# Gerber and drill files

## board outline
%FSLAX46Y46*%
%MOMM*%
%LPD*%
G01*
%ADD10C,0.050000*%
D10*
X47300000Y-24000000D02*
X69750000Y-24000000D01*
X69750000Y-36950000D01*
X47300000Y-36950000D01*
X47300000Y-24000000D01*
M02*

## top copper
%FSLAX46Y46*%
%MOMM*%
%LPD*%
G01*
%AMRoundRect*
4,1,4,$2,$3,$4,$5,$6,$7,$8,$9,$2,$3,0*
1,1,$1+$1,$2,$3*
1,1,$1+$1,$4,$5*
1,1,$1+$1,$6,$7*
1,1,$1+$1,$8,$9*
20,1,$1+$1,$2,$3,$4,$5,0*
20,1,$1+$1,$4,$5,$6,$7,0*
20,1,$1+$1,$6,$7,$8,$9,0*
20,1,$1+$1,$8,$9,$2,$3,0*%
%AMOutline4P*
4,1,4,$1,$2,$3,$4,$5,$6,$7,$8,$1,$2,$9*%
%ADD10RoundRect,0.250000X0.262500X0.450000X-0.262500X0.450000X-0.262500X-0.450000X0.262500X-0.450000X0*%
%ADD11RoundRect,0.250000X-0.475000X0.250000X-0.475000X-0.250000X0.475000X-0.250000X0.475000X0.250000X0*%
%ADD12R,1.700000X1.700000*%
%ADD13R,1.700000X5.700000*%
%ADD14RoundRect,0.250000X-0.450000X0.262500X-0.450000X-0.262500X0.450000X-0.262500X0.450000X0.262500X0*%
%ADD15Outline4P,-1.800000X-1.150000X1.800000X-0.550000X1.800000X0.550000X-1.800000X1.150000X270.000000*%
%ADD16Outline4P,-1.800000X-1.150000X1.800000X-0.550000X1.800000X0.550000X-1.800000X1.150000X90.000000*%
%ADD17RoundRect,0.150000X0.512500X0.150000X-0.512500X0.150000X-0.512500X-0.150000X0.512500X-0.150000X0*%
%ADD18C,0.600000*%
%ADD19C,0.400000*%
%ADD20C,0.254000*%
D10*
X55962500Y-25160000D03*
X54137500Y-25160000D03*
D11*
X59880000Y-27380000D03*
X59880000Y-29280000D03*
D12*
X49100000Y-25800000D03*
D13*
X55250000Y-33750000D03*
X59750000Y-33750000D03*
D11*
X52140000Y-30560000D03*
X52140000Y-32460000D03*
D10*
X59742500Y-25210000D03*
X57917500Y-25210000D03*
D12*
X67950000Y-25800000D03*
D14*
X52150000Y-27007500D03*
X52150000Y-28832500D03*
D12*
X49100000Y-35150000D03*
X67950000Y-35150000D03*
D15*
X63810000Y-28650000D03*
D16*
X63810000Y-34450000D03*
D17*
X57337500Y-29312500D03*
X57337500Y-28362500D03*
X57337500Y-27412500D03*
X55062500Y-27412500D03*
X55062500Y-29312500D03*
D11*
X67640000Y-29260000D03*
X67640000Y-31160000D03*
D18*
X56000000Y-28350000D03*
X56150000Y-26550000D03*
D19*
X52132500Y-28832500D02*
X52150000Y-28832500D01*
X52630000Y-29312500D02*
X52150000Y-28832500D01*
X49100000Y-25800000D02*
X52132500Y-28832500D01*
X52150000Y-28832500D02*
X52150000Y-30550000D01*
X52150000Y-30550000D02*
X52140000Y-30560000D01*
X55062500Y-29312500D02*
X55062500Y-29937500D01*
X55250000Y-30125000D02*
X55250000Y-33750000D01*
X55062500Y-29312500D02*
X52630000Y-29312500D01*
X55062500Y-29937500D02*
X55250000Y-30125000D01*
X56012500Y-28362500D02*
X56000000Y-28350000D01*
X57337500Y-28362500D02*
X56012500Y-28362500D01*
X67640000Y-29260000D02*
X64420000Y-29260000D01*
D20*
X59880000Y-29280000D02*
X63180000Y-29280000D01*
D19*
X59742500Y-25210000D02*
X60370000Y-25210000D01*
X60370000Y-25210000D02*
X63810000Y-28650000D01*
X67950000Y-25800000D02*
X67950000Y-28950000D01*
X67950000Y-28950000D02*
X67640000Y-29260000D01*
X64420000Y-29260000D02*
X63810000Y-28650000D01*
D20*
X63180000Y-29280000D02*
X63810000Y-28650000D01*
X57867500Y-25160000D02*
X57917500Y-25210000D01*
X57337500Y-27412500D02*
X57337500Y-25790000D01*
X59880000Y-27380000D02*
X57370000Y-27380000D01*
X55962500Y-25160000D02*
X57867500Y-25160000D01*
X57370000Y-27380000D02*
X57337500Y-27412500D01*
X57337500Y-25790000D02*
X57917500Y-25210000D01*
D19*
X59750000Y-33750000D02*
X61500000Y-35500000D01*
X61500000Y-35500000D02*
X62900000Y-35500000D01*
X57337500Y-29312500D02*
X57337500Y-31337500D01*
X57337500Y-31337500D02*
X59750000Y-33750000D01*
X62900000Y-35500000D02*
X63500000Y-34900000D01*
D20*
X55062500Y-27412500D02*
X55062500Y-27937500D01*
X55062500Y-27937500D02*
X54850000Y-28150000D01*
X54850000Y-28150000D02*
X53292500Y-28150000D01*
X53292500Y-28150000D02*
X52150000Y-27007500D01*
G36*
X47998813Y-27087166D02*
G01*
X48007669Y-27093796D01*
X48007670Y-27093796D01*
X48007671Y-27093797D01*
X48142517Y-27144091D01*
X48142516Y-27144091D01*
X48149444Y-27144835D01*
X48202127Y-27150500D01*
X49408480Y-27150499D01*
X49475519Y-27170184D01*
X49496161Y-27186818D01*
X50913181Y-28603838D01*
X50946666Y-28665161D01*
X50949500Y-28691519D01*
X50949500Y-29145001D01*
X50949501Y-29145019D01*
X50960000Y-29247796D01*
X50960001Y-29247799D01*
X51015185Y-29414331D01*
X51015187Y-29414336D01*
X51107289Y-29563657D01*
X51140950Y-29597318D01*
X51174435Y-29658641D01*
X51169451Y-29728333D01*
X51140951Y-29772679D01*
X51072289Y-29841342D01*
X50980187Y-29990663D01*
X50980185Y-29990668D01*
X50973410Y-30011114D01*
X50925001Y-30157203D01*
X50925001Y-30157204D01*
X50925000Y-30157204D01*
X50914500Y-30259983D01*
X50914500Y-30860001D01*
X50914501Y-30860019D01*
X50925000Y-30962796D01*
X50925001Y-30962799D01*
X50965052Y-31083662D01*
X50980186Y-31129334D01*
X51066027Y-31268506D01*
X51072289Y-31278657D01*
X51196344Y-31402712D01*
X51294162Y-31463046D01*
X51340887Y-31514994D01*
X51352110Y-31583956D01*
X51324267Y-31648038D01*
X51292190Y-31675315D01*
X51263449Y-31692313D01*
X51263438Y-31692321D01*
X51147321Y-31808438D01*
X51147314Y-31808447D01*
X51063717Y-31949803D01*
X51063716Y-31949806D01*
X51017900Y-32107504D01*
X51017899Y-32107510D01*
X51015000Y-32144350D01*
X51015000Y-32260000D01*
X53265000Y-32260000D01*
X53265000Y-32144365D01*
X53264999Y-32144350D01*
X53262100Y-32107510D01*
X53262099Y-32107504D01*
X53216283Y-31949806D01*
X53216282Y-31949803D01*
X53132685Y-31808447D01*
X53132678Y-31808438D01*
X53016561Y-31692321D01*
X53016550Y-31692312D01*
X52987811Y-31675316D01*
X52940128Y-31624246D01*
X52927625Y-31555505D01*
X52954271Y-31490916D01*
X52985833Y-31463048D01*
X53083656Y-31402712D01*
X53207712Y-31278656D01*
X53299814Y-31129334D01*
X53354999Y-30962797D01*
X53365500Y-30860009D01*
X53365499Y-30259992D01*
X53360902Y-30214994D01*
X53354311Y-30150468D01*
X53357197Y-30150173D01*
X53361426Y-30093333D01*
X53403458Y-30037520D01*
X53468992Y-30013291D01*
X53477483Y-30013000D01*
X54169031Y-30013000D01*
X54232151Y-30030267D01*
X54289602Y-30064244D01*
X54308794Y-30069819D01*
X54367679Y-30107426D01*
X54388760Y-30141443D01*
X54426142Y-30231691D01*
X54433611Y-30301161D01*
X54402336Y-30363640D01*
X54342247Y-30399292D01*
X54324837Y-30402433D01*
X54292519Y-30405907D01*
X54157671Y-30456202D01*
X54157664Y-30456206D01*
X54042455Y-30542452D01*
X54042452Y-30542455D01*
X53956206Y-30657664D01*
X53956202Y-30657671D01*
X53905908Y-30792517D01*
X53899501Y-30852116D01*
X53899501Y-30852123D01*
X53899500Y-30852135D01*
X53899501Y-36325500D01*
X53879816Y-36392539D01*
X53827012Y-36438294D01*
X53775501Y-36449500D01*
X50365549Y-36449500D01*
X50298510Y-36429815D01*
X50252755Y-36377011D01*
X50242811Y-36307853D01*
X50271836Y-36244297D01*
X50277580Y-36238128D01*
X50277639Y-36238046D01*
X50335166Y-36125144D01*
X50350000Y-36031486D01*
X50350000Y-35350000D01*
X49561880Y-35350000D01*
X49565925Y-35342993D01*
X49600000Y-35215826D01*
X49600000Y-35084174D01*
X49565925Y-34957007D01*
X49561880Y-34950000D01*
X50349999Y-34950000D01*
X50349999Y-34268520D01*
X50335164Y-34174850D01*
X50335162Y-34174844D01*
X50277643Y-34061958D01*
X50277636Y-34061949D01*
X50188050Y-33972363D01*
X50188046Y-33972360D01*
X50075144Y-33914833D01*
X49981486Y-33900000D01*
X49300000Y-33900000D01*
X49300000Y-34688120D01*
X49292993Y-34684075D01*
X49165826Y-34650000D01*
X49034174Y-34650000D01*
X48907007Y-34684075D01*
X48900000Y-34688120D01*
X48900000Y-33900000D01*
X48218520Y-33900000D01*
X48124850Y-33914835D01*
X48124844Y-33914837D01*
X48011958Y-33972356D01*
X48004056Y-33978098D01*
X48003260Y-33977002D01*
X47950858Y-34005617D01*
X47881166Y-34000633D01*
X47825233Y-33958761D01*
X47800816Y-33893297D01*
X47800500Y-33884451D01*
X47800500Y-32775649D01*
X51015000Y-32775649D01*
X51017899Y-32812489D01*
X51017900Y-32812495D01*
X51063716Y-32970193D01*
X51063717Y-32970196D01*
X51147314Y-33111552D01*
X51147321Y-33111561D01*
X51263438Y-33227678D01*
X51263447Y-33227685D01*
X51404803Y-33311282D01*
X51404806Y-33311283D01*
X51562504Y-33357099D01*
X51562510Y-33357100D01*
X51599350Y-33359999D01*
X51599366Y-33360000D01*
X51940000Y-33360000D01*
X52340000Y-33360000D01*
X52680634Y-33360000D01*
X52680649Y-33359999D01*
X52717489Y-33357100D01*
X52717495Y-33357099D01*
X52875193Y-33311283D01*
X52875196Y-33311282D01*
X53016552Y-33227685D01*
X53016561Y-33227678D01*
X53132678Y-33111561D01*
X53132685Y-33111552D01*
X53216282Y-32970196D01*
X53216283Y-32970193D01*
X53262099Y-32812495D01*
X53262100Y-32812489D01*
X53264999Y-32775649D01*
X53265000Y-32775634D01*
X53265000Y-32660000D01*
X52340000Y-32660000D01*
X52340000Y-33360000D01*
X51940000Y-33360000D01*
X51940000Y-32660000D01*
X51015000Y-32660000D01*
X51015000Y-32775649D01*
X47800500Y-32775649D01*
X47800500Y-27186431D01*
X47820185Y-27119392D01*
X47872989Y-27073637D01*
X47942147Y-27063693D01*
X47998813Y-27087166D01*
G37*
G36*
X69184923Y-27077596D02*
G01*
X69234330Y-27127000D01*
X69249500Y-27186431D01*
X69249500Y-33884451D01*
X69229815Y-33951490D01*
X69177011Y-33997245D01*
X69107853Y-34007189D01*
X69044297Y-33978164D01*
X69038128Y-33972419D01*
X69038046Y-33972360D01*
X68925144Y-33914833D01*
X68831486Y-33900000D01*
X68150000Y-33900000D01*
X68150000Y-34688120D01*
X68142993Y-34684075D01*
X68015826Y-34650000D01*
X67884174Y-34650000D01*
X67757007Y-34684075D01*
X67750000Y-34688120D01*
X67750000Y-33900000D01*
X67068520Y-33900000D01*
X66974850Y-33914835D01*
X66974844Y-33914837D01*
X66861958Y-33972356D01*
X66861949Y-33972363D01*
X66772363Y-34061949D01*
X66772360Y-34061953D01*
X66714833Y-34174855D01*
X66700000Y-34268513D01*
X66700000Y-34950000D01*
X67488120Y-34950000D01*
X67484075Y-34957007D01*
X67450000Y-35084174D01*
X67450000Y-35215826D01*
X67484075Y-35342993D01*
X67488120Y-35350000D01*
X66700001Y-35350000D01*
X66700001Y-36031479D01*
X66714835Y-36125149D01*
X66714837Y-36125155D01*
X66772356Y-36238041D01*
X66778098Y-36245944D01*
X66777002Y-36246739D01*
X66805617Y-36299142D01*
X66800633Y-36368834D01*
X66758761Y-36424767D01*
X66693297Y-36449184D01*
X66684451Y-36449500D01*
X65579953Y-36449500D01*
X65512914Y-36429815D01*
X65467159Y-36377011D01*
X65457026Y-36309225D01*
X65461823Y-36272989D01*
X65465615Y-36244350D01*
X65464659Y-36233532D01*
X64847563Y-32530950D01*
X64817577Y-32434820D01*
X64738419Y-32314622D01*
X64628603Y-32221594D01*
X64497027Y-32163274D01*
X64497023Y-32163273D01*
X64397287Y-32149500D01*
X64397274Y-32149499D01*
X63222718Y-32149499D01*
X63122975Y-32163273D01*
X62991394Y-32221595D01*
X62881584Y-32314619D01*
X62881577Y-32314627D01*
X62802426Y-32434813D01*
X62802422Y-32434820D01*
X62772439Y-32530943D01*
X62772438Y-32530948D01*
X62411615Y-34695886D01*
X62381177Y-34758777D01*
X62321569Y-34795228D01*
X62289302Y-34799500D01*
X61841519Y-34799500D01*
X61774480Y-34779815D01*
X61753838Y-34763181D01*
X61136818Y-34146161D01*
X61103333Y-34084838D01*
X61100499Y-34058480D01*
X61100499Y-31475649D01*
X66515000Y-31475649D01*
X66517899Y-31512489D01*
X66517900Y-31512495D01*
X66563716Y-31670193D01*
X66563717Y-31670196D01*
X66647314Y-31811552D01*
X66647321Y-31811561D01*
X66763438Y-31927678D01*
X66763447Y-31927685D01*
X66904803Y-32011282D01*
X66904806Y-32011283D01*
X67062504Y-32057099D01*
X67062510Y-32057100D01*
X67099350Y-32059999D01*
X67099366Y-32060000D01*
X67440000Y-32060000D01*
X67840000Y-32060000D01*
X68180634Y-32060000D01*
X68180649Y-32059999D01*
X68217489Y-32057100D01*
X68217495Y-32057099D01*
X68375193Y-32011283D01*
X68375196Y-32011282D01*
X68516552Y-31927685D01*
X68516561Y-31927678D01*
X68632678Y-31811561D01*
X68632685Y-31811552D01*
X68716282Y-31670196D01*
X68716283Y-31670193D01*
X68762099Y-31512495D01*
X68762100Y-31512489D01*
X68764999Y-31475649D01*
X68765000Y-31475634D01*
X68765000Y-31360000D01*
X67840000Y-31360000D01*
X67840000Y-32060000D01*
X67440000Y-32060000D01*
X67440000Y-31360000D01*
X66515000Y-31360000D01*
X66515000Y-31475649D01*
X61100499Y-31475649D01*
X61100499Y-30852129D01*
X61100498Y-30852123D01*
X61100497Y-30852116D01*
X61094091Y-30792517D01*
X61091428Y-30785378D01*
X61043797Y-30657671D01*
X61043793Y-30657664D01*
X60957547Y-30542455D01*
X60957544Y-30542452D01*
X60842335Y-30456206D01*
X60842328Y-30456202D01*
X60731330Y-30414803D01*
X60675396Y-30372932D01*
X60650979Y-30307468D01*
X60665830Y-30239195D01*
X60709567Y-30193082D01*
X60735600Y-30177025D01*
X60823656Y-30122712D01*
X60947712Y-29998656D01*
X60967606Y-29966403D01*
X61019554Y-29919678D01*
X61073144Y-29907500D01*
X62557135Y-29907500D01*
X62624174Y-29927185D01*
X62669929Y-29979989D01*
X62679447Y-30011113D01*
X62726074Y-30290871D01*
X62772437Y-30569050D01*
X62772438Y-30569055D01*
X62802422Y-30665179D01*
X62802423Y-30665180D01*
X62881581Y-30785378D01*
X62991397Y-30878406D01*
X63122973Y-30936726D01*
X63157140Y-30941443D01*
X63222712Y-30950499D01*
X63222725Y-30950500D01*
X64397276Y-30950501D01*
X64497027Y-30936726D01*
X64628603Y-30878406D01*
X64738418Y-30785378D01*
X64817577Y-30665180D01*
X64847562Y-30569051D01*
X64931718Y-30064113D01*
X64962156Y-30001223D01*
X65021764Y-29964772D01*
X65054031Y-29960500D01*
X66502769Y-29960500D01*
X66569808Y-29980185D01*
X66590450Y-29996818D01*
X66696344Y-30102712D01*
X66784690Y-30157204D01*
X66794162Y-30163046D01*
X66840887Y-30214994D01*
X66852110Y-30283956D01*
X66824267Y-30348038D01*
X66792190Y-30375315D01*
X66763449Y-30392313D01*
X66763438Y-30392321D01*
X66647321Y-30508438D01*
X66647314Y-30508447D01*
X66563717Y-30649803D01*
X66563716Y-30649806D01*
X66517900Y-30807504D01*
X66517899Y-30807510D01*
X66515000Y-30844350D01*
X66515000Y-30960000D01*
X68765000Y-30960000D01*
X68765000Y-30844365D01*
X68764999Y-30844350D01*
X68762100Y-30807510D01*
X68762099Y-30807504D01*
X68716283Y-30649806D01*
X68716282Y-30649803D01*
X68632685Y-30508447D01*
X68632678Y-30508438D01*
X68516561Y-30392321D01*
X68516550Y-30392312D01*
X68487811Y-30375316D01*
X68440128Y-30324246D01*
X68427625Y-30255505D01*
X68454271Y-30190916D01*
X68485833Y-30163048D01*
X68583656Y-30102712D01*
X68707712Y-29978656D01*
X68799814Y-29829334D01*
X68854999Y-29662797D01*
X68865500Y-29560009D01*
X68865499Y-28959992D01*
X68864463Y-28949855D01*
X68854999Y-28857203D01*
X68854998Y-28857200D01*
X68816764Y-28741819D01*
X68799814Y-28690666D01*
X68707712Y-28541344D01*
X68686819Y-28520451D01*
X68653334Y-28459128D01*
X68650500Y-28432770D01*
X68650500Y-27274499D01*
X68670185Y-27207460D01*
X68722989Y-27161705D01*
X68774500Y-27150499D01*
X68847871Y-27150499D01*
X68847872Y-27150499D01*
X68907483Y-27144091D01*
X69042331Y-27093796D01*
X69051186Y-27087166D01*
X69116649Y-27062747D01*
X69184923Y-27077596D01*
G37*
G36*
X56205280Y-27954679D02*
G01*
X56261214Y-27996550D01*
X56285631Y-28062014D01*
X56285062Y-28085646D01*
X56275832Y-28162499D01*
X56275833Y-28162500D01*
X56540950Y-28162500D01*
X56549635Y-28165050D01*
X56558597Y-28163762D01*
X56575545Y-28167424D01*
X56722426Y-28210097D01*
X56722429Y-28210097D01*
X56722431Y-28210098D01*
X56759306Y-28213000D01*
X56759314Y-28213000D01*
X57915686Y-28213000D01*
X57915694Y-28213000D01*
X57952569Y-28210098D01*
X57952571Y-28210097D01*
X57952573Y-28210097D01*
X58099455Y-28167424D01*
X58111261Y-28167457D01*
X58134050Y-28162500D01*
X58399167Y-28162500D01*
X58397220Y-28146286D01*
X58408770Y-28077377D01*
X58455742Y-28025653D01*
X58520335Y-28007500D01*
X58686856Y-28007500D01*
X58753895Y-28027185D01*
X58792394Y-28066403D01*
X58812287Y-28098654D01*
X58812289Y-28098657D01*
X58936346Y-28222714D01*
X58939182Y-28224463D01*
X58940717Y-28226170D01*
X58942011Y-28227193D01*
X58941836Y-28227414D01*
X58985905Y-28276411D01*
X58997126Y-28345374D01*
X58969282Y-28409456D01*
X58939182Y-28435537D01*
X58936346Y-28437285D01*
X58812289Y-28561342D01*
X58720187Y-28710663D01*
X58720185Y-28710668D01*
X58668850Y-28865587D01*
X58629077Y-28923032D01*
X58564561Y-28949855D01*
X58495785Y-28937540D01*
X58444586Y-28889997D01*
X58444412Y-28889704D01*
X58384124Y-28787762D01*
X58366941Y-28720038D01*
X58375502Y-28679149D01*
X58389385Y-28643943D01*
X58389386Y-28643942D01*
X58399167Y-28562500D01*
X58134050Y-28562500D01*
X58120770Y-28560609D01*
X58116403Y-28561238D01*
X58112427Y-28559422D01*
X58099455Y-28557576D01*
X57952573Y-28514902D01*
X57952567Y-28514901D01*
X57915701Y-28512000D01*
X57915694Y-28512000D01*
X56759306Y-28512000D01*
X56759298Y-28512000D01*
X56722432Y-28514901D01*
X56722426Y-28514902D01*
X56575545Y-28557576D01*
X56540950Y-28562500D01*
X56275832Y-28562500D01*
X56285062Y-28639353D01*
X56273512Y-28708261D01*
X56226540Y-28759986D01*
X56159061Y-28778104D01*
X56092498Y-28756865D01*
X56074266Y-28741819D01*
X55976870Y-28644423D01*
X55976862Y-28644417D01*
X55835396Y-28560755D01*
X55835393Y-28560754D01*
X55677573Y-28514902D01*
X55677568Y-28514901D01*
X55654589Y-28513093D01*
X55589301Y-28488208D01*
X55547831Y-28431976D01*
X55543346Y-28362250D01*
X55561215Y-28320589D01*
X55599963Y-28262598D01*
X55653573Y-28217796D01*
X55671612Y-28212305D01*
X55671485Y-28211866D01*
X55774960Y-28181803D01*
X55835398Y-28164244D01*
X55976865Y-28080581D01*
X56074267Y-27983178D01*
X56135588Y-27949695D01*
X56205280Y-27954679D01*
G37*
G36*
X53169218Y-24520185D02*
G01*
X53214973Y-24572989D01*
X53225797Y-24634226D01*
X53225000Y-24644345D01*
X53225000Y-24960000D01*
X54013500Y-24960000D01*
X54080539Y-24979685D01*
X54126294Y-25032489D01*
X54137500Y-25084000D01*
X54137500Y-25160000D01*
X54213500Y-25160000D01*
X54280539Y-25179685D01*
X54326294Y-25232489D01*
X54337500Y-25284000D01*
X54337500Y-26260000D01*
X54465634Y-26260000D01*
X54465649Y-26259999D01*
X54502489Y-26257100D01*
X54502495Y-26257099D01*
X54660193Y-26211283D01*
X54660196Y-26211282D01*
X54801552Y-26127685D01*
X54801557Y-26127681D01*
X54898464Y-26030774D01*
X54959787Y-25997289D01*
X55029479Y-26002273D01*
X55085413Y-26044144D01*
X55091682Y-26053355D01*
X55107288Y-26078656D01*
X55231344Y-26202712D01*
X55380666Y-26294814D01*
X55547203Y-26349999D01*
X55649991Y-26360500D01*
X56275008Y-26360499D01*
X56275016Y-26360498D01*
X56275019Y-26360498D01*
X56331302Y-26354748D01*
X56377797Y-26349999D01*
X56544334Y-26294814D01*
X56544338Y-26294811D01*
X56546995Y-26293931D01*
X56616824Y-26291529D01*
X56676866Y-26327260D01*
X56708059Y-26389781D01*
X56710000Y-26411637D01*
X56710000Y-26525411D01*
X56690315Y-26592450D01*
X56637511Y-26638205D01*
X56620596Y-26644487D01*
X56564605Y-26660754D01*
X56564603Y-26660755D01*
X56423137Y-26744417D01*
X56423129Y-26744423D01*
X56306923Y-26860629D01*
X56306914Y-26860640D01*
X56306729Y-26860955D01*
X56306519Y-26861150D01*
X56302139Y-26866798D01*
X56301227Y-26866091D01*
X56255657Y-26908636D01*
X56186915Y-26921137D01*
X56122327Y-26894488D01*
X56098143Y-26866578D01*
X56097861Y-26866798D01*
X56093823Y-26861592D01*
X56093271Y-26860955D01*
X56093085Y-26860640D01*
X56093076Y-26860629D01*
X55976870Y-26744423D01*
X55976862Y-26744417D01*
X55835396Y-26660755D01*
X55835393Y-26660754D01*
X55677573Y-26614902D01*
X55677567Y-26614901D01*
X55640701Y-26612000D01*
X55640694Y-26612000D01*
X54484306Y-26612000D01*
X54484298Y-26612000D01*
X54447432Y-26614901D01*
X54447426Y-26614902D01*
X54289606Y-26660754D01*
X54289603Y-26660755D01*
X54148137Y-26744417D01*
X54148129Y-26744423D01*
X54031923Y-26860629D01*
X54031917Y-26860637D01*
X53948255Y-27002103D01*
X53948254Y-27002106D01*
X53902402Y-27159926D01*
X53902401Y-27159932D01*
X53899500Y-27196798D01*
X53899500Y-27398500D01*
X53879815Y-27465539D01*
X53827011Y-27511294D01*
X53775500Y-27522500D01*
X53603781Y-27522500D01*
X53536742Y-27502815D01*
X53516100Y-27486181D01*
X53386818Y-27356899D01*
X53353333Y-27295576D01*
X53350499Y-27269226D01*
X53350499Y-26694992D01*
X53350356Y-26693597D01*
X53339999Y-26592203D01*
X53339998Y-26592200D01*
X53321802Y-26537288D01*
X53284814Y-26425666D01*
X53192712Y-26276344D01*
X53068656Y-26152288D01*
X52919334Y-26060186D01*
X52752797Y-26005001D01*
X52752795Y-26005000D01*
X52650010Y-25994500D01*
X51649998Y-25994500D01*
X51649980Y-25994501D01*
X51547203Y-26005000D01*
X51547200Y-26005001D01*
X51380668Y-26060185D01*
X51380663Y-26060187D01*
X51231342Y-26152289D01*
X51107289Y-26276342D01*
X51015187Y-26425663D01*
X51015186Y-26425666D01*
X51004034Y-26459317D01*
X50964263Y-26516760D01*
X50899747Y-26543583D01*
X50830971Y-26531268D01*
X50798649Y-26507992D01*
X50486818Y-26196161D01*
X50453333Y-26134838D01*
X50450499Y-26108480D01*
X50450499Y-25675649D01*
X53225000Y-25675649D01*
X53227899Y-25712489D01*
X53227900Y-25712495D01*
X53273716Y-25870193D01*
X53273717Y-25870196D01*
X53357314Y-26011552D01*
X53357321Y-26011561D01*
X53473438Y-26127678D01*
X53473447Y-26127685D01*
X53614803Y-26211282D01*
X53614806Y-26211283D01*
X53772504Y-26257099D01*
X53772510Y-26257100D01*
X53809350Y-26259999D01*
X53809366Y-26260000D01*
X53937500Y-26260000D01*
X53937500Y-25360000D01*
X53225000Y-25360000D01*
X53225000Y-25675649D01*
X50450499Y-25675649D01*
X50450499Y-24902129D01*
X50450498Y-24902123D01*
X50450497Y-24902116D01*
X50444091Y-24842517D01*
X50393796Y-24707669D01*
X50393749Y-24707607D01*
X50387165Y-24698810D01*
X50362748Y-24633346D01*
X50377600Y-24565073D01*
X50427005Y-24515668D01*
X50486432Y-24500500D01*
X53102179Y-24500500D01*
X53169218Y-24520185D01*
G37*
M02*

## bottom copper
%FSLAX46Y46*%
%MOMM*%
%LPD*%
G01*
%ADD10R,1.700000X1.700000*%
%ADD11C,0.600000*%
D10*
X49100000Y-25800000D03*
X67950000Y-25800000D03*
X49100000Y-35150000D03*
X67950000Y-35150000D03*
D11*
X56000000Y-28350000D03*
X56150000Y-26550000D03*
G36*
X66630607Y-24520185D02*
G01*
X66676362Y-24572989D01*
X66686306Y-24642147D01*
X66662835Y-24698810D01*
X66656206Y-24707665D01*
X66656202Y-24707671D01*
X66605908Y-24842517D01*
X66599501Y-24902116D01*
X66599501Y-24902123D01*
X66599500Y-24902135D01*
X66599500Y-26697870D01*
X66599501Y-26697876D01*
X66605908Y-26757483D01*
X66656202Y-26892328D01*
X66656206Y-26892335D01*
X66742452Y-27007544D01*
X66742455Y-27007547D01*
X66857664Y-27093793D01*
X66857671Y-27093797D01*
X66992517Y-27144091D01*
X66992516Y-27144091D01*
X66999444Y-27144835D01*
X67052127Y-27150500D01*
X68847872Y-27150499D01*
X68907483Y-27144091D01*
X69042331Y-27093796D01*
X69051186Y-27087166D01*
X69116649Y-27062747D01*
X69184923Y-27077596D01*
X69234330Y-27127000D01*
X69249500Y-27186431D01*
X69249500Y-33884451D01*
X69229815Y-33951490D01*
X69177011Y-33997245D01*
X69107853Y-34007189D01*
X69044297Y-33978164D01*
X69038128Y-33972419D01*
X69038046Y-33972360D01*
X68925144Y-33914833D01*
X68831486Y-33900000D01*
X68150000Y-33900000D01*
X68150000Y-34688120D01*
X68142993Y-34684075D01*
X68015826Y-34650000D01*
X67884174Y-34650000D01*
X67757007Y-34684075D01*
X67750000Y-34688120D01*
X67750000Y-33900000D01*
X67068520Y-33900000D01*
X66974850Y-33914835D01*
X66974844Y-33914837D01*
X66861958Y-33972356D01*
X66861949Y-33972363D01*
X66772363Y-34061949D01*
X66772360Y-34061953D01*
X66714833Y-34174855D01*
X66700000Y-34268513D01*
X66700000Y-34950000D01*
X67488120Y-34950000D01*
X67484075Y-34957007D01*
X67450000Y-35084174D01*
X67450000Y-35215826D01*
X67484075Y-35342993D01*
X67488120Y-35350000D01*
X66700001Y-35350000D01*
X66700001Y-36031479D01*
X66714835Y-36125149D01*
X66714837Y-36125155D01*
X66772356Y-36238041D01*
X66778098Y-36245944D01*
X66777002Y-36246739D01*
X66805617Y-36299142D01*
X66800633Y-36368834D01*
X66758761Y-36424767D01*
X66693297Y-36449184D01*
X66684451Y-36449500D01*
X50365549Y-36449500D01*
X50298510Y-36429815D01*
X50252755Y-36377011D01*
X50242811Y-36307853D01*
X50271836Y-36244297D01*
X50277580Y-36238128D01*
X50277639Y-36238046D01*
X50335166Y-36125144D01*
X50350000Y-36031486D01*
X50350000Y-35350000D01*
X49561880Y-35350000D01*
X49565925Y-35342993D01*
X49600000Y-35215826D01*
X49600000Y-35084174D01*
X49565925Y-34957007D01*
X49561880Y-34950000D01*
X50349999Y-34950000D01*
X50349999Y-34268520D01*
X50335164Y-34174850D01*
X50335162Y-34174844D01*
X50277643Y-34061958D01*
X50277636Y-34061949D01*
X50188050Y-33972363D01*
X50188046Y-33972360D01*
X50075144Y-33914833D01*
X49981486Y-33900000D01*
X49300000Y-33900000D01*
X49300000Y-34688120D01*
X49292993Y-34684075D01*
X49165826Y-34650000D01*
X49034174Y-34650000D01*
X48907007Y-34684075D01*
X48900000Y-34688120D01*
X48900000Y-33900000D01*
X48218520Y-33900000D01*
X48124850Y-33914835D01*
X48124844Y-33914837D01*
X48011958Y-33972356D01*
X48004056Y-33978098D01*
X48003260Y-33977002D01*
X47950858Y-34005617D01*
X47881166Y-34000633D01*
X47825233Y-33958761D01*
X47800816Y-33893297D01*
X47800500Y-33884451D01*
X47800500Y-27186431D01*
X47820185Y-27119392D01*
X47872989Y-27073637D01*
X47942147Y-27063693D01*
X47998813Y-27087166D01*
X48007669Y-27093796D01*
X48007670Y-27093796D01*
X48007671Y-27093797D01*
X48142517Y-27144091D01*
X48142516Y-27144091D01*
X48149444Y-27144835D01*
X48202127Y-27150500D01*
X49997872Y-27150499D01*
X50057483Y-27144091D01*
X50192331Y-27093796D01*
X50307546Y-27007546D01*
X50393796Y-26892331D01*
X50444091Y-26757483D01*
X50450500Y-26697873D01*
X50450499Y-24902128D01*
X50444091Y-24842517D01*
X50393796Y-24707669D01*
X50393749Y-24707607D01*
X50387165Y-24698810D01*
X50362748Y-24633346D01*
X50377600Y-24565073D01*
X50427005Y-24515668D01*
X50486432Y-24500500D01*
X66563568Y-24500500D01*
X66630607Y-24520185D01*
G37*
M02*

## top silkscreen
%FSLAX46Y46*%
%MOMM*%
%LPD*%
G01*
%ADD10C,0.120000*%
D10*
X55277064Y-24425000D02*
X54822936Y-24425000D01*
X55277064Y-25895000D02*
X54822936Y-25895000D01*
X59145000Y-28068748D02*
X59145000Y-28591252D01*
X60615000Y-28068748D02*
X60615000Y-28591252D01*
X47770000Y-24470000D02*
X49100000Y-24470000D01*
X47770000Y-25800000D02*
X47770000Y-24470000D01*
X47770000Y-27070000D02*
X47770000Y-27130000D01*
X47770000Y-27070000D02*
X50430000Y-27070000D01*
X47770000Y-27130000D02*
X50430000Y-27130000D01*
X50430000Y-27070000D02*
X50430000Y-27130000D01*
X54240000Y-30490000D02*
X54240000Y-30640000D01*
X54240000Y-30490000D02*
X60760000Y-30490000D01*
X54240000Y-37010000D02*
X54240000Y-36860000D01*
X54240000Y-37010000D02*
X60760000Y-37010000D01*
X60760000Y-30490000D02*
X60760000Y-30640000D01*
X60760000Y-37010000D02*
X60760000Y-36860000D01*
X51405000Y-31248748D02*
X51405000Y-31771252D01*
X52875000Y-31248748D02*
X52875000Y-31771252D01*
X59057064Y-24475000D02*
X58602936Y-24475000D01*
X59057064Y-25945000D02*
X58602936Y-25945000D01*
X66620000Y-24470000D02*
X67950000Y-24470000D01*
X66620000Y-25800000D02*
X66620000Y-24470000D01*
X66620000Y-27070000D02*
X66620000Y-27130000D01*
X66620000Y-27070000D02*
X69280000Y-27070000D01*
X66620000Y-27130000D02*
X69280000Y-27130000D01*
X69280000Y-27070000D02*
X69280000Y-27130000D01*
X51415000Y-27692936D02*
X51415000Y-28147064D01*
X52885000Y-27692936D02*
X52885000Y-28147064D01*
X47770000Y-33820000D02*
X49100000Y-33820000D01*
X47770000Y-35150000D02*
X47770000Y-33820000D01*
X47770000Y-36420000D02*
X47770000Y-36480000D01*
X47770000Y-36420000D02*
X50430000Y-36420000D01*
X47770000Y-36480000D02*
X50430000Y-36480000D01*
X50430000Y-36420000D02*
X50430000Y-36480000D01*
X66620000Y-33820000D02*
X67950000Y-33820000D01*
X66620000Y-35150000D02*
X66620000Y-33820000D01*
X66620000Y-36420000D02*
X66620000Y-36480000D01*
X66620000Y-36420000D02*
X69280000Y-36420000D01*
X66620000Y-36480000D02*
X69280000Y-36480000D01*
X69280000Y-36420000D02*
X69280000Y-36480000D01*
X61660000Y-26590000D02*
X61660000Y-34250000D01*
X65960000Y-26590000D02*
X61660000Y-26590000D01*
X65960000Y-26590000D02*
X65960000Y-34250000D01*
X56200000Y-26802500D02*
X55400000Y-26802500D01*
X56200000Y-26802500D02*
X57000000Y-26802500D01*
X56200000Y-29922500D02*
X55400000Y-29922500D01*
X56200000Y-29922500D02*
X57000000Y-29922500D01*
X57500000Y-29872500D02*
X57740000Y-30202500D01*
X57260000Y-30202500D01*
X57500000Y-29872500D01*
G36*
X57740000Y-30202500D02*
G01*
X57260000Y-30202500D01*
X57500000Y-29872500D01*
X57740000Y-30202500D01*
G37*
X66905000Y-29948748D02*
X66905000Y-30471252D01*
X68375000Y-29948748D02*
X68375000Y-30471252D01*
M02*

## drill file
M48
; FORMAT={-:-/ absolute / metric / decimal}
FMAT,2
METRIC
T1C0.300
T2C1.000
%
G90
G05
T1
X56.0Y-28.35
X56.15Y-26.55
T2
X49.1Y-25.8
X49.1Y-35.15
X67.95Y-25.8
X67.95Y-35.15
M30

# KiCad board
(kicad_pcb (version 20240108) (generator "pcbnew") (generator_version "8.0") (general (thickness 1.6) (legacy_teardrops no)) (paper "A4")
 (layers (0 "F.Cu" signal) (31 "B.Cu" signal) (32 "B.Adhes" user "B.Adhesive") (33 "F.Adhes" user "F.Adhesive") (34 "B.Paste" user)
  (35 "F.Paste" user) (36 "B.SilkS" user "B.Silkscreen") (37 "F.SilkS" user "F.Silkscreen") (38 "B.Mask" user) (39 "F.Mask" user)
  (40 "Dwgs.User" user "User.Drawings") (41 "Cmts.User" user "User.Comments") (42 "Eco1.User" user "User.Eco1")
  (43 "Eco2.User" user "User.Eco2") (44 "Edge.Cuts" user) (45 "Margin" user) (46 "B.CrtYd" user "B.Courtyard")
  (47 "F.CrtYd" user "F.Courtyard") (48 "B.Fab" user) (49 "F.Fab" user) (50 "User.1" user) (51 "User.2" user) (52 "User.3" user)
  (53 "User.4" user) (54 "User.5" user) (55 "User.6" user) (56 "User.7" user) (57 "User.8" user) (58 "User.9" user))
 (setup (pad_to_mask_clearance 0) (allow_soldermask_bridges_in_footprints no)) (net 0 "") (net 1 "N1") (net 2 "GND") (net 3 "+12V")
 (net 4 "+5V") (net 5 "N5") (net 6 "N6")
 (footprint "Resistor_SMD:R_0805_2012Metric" (layer "F.Cu") (at 55.05 25.16 180)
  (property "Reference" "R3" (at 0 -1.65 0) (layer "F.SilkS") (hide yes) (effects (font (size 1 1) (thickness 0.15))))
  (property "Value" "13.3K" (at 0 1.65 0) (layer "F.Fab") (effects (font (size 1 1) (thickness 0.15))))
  (fp_line (start -0.227064 0.735) (end 0.227064 0.735) (stroke (width 0.12) (type solid)) (layer "F.SilkS"))
  (fp_line (start -0.227064 -0.735) (end 0.227064 -0.735) (stroke (width 0.12) (type solid)) (layer "F.SilkS"))
  (pad "1" smd roundrect (at -0.9125 0 180) (size 1.025 1.4) (layers "F.Cu" "F.Paste" "F.Mask") (roundrect_rratio 0.243902) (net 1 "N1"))
  (pad "2" smd roundrect (at 0.9125 0 180) (size 1.025 1.4) (layers "F.Cu" "F.Paste" "F.Mask") (roundrect_rratio 0.243902) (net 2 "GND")))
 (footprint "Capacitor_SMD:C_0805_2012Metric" (layer "F.Cu") (at 59.88 28.33 -90)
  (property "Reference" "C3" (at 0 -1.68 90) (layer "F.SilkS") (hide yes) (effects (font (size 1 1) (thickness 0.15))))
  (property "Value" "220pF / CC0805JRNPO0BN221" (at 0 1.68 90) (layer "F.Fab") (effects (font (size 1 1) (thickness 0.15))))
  (fp_line (start -0.261252 0.735) (end 0.261252 0.735) (stroke (width 0.12) (type solid)) (layer "F.SilkS"))
  (fp_line (start -0.261252 -0.735) (end 0.261252 -0.735) (stroke (width 0.12) (type solid)) (layer "F.SilkS"))
  (pad "1" smd roundrect (at -0.95 0 270) (size 1 1.45) (layers "F.Cu" "F.Paste" "F.Mask") (roundrect_rratio 0.25) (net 1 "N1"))
  (pad "2" smd roundrect (at 0.95 0 270) (size 1 1.45) (layers "F.Cu" "F.Paste" "F.Mask") (roundrect_rratio 0.25) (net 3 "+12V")))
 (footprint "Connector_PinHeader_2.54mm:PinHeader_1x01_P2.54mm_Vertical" (layer "F.Cu") (at 49.1 25.8)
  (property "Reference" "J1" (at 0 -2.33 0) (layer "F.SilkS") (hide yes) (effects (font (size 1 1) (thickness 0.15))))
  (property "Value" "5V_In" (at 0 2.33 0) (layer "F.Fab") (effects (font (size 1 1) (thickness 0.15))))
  (fp_line (start -1.33 -1.33) (end 0 -1.33) (stroke (width 0.12) (type solid)) (layer "F.SilkS"))
  (fp_line (start -1.33 0) (end -1.33 -1.33) (stroke (width 0.12) (type solid)) (layer "F.SilkS"))
  (fp_line (start -1.33 1.27) (end -1.33 1.33) (stroke (width 0.12) (type solid)) (layer "F.SilkS"))
  (fp_line (start -1.33 1.27) (end 1.33 1.27) (stroke (width 0.12) (type solid)) (layer "F.SilkS"))
  (fp_line (start -1.33 1.33) (end 1.33 1.33) (stroke (width 0.12) (type solid)) (layer "F.SilkS"))
  (fp_line (start 1.33 1.27) (end 1.33 1.33) (stroke (width 0.12) (type solid)) (layer "F.SilkS"))
  (pad "1" thru_hole rect (at 0 0) (size 1.7 1.7) (drill 1) (layers "*.Cu" "*.Mask") (remove_unused_layers no) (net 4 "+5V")))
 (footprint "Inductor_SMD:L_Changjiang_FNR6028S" (layer "F.Cu") (at 57.5 33.75)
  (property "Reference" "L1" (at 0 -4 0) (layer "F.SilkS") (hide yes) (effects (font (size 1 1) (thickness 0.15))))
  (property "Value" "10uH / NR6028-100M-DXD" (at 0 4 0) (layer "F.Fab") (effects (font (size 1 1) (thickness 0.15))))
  (fp_line (start -3.26 -3.26) (end -3.26 -3.11) (stroke (width 0.12) (type solid)) (layer "F.SilkS"))
  (fp_line (start -3.26 -3.26) (end 3.26 -3.26) (stroke (width 0.12) (type solid)) (layer "F.SilkS"))
  (fp_line (start -3.26 3.26) (end -3.26 3.11) (stroke (width 0.12) (type solid)) (layer "F.SilkS"))
  (fp_line (start -3.26 3.26) (end 3.26 3.26) (stroke (width 0.12) (type solid)) (layer "F.SilkS"))
  (fp_line (start 3.26 -3.26) (end 3.26 -3.11) (stroke (width 0.12) (type solid)) (layer "F.SilkS"))
  (fp_line (start 3.26 3.26) (end 3.26 3.11) (stroke (width 0.12) (type solid)) (layer "F.SilkS"))
  (pad "1" smd rect (at -2.25 0) (size 1.7 5.7) (layers "F.Cu" "F.Paste" "F.Mask") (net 4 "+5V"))
  (pad "2" smd rect (at 2.25 0) (size 1.7 5.7) (layers "F.Cu" "F.Paste" "F.Mask") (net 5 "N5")))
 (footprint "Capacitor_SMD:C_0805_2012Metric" (layer "F.Cu") (at 52.14 31.51 -90)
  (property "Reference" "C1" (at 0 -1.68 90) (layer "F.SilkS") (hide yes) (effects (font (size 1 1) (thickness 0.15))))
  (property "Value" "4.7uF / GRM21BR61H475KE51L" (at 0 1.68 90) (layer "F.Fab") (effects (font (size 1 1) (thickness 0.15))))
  (fp_line (start -0.261252 0.735) (end 0.261252 0.735) (stroke (width 0.12) (type solid)) (layer "F.SilkS"))
  (fp_line (start -0.261252 -0.735) (end 0.261252 -0.735) (stroke (width 0.12) (type solid)) (layer "F.SilkS"))
  (pad "1" smd roundrect (at -0.95 0 270) (size 1 1.45) (layers "F.Cu" "F.Paste" "F.Mask") (roundrect_rratio 0.25) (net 4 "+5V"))
  (pad "2" smd roundrect (at 0.95 0 270) (size 1 1.45) (layers "F.Cu" "F.Paste" "F.Mask") (roundrect_rratio 0.25) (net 2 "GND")))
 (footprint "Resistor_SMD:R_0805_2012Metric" (layer "F.Cu") (at 58.83 25.21 180)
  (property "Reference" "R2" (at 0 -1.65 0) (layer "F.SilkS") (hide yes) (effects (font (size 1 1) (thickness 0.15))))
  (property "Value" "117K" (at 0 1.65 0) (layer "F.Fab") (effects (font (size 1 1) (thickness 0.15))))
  (fp_line (start -0.227064 0.735) (end 0.227064 0.735) (stroke (width 0.12) (type solid)) (layer "F.SilkS"))
  (fp_line (start -0.227064 -0.735) (end 0.227064 -0.735) (stroke (width 0.12) (type solid)) (layer "F.SilkS"))
  (pad "1" smd roundrect (at -0.9125 0 180) (size 1.025 1.4) (layers "F.Cu" "F.Paste" "F.Mask") (roundrect_rratio 0.243902) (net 3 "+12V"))
  (pad "2" smd roundrect (at 0.9125 0 180) (size 1.025 1.4) (layers "F.Cu" "F.Paste" "F.Mask") (roundrect_rratio 0.243902) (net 1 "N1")))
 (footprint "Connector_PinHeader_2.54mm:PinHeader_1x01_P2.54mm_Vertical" (layer "F.Cu") (at 67.95 25.8)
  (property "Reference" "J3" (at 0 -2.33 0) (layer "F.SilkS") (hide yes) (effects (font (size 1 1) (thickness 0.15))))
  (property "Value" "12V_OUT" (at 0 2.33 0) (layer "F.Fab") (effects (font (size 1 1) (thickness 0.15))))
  (fp_line (start -1.33 -1.33) (end 0 -1.33) (stroke (width 0.12) (type solid)) (layer "F.SilkS"))
  (fp_line (start -1.33 0) (end -1.33 -1.33) (stroke (width 0.12) (type solid)) (layer "F.SilkS"))
  (fp_line (start -1.33 1.27) (end -1.33 1.33) (stroke (width 0.12) (type solid)) (layer "F.SilkS"))
  (fp_line (start -1.33 1.27) (end 1.33 1.27) (stroke (width 0.12) (type solid)) (layer "F.SilkS"))
  (fp_line (start -1.33 1.33) (end 1.33 1.33) (stroke (width 0.12) (type solid)) (layer "F.SilkS"))
  (fp_line (start 1.33 1.27) (end 1.33 1.33) (stroke (width 0.12) (type solid)) (layer "F.SilkS"))
  (pad "1" thru_hole rect (at 0 0) (size 1.7 1.7) (drill 1) (layers "*.Cu" "*.Mask") (remove_unused_layers no) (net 3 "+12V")))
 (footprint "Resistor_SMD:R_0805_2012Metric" (layer "F.Cu") (at 52.15 27.92 -90)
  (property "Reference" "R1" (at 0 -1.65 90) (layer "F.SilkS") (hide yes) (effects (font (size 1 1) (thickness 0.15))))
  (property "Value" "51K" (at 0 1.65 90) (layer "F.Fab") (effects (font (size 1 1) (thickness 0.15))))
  (fp_line (start -0.227064 0.735) (end 0.227064 0.735) (stroke (width 0.12) (type solid)) (layer "F.SilkS"))
  (fp_line (start -0.227064 -0.735) (end 0.227064 -0.735) (stroke (width 0.12) (type solid)) (layer "F.SilkS"))
  (pad "1" smd roundrect (at -0.9125 0 270) (size 1.025 1.4) (layers "F.Cu" "F.Paste" "F.Mask") (roundrect_rratio 0.243902) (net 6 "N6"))
  (pad "2" smd roundrect (at 0.9125 0 270) (size 1.025 1.4) (layers "F.Cu" "F.Paste" "F.Mask") (roundrect_rratio 0.243902) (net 4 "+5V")))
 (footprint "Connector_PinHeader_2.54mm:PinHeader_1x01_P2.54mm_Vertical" (layer "F.Cu") (at 49.1 35.15)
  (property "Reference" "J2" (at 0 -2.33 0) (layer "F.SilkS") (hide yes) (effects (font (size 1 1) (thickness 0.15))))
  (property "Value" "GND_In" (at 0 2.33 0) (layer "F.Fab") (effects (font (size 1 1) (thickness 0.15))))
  (fp_line (start -1.33 -1.33) (end 0 -1.33) (stroke (width 0.12) (type solid)) (layer "F.SilkS"))
  (fp_line (start -1.33 0) (end -1.33 -1.33) (stroke (width 0.12) (type solid)) (layer "F.SilkS"))
  (fp_line (start -1.33 1.27) (end -1.33 1.33) (stroke (width 0.12) (type solid)) (layer "F.SilkS"))
  (fp_line (start -1.33 1.27) (end 1.33 1.27) (stroke (width 0.12) (type solid)) (layer "F.SilkS"))
  (fp_line (start -1.33 1.33) (end 1.33 1.33) (stroke (width 0.12) (type solid)) (layer "F.SilkS"))
  (fp_line (start 1.33 1.27) (end 1.33 1.33) (stroke (width 0.12) (type solid)) (layer "F.SilkS"))
  (pad "1" thru_hole rect (at 0 0) (size 1.7 1.7) (drill 1) (layers "*.Cu" "*.Mask") (remove_unused_layers no) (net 2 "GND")))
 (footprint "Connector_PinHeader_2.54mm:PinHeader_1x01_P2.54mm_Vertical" (layer "F.Cu") (at 67.95 35.15)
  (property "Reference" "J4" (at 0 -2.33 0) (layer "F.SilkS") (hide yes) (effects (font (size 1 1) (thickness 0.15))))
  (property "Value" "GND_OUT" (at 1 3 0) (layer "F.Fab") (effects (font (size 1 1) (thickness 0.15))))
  (fp_line (start -1.33 -1.33) (end 0 -1.33) (stroke (width 0.12) (type solid)) (layer "F.SilkS"))
  (fp_line (start -1.33 0) (end -1.33 -1.33) (stroke (width 0.12) (type solid)) (layer "F.SilkS"))
  (fp_line (start -1.33 1.27) (end -1.33 1.33) (stroke (width 0.12) (type solid)) (layer "F.SilkS"))
  (fp_line (start -1.33 1.27) (end 1.33 1.27) (stroke (width 0.12) (type solid)) (layer "F.SilkS"))
  (fp_line (start -1.33 1.33) (end 1.33 1.33) (stroke (width 0.12) (type solid)) (layer "F.SilkS"))
  (fp_line (start 1.33 1.27) (end 1.33 1.33) (stroke (width 0.12) (type solid)) (layer "F.SilkS"))
  (pad "1" thru_hole rect (at 0 0) (size 1.7 1.7) (drill 1) (layers "*.Cu" "*.Mask") (remove_unused_layers no) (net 2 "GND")))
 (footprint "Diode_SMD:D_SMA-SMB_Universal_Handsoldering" (layer "F.Cu") (at 63.81 31.55 -90)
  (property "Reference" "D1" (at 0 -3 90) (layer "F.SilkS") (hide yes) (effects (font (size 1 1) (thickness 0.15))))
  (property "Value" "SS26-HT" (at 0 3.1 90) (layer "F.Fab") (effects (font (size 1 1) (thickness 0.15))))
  (fp_line (start -4.96 2.15) (end 2.7 2.15) (stroke (width 0.12) (type solid)) (layer "F.SilkS"))
  (fp_line (start -4.96 -2.15) (end -4.96 2.15) (stroke (width 0.12) (type solid)) (layer "F.SilkS"))
  (fp_line (start -4.96 -2.15) (end 2.7 -2.15) (stroke (width 0.12) (type solid)) (layer "F.SilkS"))
  (pad "1" smd trapezoid (at -2.9 0 270) (size 3.6 1.7) (rect_delta 0.6 0) (layers "F.Cu" "F.Paste" "F.Mask") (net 3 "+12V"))
  (pad "2" smd trapezoid (at 2.9 0 90) (size 3.6 1.7) (rect_delta 0.6 0) (layers "F.Cu" "F.Paste" "F.Mask") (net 5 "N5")))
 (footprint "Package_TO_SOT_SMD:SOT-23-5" (layer "F.Cu") (at 56.2 28.3625 180)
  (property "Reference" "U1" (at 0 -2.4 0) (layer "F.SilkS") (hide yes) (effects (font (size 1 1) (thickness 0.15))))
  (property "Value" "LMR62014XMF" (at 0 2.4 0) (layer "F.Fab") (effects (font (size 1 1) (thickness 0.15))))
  (fp_line (start 0 1.56) (end 0.8 1.56) (stroke (width 0.12) (type solid)) (layer "F.SilkS"))
  (fp_line (start 0 1.56) (end -0.8 1.56) (stroke (width 0.12) (type solid)) (layer "F.SilkS"))
  (fp_line (start 0 -1.56) (end 0.8 -1.56) (stroke (width 0.12) (type solid)) (layer "F.SilkS"))
  (fp_line (start 0 -1.56) (end -0.8 -1.56) (stroke (width 0.12) (type solid)) (layer "F.SilkS"))
  (fp_poly
   (pts (xy -1.3 -1.51) (xy -1.54 -1.84) (xy -1.06 -1.84) (xy -1.3 -1.51)) (stroke (width 0.12) (type solid)) (fill solid) (layer "F.SilkS"))
  (pad "1" smd roundrect (at -1.1375 -0.95 180) (size 1.325 0.6) (layers "F.Cu" "F.Paste" "F.Mask") (roundrect_rratio 0.25) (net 5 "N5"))
  (pad "2" smd roundrect (at -1.1375 0 180) (size 1.325 0.6) (layers "F.Cu" "F.Paste" "F.Mask") (roundrect_rratio 0.25) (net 2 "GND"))
  (pad "3" smd roundrect (at -1.1375 0.95 180) (size 1.325 0.6) (layers "F.Cu" "F.Paste" "F.Mask") (roundrect_rratio 0.25) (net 1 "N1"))
  (pad "4" smd roundrect (at 1.1375 0.95 180) (size 1.325 0.6) (layers "F.Cu" "F.Paste" "F.Mask") (roundrect_rratio 0.25) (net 6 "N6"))
  (pad "5" smd roundrect (at 1.1375 -0.95 180) (size 1.325 0.6) (layers "F.Cu" "F.Paste" "F.Mask") (roundrect_rratio 0.25) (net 4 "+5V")))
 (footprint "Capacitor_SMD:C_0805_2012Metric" (layer "F.Cu") (at 67.64 30.21 -90)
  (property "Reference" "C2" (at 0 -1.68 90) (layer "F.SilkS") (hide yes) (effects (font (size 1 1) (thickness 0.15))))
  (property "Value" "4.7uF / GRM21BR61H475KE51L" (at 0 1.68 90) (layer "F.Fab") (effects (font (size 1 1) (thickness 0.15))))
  (fp_line (start -0.261252 0.735) (end 0.261252 0.735) (stroke (width 0.12) (type solid)) (layer "F.SilkS"))
  (fp_line (start -0.261252 -0.735) (end 0.261252 -0.735) (stroke (width 0.12) (type solid)) (layer "F.SilkS"))
  (pad "1" smd roundrect (at -0.95 0 270) (size 1 1.45) (layers "F.Cu" "F.Paste" "F.Mask") (roundrect_rratio 0.25) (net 3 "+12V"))
  (pad "2" smd roundrect (at 0.95 0 270) (size 1 1.45) (layers "F.Cu" "F.Paste" "F.Mask") (roundrect_rratio 0.25) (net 2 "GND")))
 (gr_rect (start 47.3 24) (end 69.75 36.95) (stroke (width 0.05) (type default)) (fill none) (layer "Edge.Cuts"))
 (segment (start 52.1325 28.8325) (end 52.15 28.8325) (width 0.4) (layer "F.Cu") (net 4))
 (segment (start 52.63 29.3125) (end 52.15 28.8325) (width 0.4) (layer "F.Cu") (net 4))
 (segment (start 49.1 25.8) (end 52.1325 28.8325) (width 0.4) (layer "F.Cu") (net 4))
 (segment (start 52.15 28.8325) (end 52.15 30.55) (width 0.4) (layer "F.Cu") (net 4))
 (segment (start 52.15 30.55) (end 52.14 30.56) (width 0.4) (layer "F.Cu") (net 4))
 (segment (start 55.0625 29.3125) (end 55.0625 29.9375) (width 0.4) (layer "F.Cu") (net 4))
 (segment (start 55.25 30.125) (end 55.25 33.75) (width 0.4) (layer "F.Cu") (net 4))
 (segment (start 55.0625 29.3125) (end 52.63 29.3125) (width 0.4) (layer "F.Cu") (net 4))
 (segment (start 55.0625 29.9375) (end 55.25 30.125) (width 0.4) (layer "F.Cu") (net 4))
 (segment (start 56.0125 28.3625) (end 56 28.35) (width 0.4) (layer "F.Cu") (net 2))
 (segment (start 57.3375 28.3625) (end 56.0125 28.3625) (width 0.4) (layer "F.Cu") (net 2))
 (via (at 56 28.35) (size 0.6) (drill 0.3) (layers "F.Cu" "B.Cu") (free yes) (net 2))
 (via (at 56.15 26.55) (size 0.6) (drill 0.3) (layers "F.Cu" "B.Cu") (free yes) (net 2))
 (segment (start 67.64 29.26) (end 64.42 29.26) (width 0.4) (layer "F.Cu") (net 3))
 (segment (start 59.88 29.28) (end 63.18 29.28) (width 0.254) (layer "F.Cu") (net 3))
 (segment (start 59.7425 25.21) (end 60.37 25.21) (width 0.4) (layer "F.Cu") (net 3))
 (segment (start 60.37 25.21) (end 63.81 28.65) (width 0.4) (layer "F.Cu") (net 3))
 (segment (start 67.95 25.8) (end 67.95 28.95) (width 0.4) (layer "F.Cu") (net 3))
 (segment (start 67.95 28.95) (end 67.64 29.26) (width 0.4) (layer "F.Cu") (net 3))
 (segment (start 64.42 29.26) (end 63.81 28.65) (width 0.4) (layer "F.Cu") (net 3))
 (segment (start 63.18 29.28) (end 63.81 28.65) (width 0.254) (layer "F.Cu") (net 3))
 (segment (start 57.8675 25.16) (end 57.9175 25.21) (width 0.254) (layer "F.Cu") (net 1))
 (segment (start 57.3375 27.4125) (end 57.3375 25.79) (width 0.254) (layer "F.Cu") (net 1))
 (segment (start 59.88 27.38) (end 57.37 27.38) (width 0.254) (layer "F.Cu") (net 1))
 (segment (start 55.9625 25.16) (end 57.8675 25.16) (width 0.254) (layer "F.Cu") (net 1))
 (segment (start 57.37 27.38) (end 57.3375 27.4125) (width 0.254) (layer "F.Cu") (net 1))
 (segment (start 57.3375 25.79) (end 57.9175 25.21) (width 0.254) (layer "F.Cu") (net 1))
 (segment (start 59.75 33.75) (end 61.5 35.5) (width 0.4) (layer "F.Cu") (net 5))
 (segment (start 61.5 35.5) (end 62.9 35.5) (width 0.4) (layer "F.Cu") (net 5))
 (segment (start 57.3375 29.3125) (end 57.3375 31.3375) (width 0.4) (layer "F.Cu") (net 5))
 (segment (start 57.3375 31.3375) (end 59.75 33.75) (width 0.4) (layer "F.Cu") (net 5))
 (segment (start 62.9 35.5) (end 63.5 34.9) (width 0.4) (layer "F.Cu") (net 5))
 (segment (start 55.0625 27.4125) (end 55.0625 27.9375) (width 0.254) (layer "F.Cu") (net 6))
 (segment (start 55.0625 27.9375) (end 54.85 28.15) (width 0.254) (layer "F.Cu") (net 6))
 (segment (start 54.85 28.15) (end 53.2925 28.15) (width 0.254) (layer "F.Cu") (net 6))
 (segment (start 53.2925 28.15) (end 52.15 27.0075) (width 0.254) (layer "F.Cu") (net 6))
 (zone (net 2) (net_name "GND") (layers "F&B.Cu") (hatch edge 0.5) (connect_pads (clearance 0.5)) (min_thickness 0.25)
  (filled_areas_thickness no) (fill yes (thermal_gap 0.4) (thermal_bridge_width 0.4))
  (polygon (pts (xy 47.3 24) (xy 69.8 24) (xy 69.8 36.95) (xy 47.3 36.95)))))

